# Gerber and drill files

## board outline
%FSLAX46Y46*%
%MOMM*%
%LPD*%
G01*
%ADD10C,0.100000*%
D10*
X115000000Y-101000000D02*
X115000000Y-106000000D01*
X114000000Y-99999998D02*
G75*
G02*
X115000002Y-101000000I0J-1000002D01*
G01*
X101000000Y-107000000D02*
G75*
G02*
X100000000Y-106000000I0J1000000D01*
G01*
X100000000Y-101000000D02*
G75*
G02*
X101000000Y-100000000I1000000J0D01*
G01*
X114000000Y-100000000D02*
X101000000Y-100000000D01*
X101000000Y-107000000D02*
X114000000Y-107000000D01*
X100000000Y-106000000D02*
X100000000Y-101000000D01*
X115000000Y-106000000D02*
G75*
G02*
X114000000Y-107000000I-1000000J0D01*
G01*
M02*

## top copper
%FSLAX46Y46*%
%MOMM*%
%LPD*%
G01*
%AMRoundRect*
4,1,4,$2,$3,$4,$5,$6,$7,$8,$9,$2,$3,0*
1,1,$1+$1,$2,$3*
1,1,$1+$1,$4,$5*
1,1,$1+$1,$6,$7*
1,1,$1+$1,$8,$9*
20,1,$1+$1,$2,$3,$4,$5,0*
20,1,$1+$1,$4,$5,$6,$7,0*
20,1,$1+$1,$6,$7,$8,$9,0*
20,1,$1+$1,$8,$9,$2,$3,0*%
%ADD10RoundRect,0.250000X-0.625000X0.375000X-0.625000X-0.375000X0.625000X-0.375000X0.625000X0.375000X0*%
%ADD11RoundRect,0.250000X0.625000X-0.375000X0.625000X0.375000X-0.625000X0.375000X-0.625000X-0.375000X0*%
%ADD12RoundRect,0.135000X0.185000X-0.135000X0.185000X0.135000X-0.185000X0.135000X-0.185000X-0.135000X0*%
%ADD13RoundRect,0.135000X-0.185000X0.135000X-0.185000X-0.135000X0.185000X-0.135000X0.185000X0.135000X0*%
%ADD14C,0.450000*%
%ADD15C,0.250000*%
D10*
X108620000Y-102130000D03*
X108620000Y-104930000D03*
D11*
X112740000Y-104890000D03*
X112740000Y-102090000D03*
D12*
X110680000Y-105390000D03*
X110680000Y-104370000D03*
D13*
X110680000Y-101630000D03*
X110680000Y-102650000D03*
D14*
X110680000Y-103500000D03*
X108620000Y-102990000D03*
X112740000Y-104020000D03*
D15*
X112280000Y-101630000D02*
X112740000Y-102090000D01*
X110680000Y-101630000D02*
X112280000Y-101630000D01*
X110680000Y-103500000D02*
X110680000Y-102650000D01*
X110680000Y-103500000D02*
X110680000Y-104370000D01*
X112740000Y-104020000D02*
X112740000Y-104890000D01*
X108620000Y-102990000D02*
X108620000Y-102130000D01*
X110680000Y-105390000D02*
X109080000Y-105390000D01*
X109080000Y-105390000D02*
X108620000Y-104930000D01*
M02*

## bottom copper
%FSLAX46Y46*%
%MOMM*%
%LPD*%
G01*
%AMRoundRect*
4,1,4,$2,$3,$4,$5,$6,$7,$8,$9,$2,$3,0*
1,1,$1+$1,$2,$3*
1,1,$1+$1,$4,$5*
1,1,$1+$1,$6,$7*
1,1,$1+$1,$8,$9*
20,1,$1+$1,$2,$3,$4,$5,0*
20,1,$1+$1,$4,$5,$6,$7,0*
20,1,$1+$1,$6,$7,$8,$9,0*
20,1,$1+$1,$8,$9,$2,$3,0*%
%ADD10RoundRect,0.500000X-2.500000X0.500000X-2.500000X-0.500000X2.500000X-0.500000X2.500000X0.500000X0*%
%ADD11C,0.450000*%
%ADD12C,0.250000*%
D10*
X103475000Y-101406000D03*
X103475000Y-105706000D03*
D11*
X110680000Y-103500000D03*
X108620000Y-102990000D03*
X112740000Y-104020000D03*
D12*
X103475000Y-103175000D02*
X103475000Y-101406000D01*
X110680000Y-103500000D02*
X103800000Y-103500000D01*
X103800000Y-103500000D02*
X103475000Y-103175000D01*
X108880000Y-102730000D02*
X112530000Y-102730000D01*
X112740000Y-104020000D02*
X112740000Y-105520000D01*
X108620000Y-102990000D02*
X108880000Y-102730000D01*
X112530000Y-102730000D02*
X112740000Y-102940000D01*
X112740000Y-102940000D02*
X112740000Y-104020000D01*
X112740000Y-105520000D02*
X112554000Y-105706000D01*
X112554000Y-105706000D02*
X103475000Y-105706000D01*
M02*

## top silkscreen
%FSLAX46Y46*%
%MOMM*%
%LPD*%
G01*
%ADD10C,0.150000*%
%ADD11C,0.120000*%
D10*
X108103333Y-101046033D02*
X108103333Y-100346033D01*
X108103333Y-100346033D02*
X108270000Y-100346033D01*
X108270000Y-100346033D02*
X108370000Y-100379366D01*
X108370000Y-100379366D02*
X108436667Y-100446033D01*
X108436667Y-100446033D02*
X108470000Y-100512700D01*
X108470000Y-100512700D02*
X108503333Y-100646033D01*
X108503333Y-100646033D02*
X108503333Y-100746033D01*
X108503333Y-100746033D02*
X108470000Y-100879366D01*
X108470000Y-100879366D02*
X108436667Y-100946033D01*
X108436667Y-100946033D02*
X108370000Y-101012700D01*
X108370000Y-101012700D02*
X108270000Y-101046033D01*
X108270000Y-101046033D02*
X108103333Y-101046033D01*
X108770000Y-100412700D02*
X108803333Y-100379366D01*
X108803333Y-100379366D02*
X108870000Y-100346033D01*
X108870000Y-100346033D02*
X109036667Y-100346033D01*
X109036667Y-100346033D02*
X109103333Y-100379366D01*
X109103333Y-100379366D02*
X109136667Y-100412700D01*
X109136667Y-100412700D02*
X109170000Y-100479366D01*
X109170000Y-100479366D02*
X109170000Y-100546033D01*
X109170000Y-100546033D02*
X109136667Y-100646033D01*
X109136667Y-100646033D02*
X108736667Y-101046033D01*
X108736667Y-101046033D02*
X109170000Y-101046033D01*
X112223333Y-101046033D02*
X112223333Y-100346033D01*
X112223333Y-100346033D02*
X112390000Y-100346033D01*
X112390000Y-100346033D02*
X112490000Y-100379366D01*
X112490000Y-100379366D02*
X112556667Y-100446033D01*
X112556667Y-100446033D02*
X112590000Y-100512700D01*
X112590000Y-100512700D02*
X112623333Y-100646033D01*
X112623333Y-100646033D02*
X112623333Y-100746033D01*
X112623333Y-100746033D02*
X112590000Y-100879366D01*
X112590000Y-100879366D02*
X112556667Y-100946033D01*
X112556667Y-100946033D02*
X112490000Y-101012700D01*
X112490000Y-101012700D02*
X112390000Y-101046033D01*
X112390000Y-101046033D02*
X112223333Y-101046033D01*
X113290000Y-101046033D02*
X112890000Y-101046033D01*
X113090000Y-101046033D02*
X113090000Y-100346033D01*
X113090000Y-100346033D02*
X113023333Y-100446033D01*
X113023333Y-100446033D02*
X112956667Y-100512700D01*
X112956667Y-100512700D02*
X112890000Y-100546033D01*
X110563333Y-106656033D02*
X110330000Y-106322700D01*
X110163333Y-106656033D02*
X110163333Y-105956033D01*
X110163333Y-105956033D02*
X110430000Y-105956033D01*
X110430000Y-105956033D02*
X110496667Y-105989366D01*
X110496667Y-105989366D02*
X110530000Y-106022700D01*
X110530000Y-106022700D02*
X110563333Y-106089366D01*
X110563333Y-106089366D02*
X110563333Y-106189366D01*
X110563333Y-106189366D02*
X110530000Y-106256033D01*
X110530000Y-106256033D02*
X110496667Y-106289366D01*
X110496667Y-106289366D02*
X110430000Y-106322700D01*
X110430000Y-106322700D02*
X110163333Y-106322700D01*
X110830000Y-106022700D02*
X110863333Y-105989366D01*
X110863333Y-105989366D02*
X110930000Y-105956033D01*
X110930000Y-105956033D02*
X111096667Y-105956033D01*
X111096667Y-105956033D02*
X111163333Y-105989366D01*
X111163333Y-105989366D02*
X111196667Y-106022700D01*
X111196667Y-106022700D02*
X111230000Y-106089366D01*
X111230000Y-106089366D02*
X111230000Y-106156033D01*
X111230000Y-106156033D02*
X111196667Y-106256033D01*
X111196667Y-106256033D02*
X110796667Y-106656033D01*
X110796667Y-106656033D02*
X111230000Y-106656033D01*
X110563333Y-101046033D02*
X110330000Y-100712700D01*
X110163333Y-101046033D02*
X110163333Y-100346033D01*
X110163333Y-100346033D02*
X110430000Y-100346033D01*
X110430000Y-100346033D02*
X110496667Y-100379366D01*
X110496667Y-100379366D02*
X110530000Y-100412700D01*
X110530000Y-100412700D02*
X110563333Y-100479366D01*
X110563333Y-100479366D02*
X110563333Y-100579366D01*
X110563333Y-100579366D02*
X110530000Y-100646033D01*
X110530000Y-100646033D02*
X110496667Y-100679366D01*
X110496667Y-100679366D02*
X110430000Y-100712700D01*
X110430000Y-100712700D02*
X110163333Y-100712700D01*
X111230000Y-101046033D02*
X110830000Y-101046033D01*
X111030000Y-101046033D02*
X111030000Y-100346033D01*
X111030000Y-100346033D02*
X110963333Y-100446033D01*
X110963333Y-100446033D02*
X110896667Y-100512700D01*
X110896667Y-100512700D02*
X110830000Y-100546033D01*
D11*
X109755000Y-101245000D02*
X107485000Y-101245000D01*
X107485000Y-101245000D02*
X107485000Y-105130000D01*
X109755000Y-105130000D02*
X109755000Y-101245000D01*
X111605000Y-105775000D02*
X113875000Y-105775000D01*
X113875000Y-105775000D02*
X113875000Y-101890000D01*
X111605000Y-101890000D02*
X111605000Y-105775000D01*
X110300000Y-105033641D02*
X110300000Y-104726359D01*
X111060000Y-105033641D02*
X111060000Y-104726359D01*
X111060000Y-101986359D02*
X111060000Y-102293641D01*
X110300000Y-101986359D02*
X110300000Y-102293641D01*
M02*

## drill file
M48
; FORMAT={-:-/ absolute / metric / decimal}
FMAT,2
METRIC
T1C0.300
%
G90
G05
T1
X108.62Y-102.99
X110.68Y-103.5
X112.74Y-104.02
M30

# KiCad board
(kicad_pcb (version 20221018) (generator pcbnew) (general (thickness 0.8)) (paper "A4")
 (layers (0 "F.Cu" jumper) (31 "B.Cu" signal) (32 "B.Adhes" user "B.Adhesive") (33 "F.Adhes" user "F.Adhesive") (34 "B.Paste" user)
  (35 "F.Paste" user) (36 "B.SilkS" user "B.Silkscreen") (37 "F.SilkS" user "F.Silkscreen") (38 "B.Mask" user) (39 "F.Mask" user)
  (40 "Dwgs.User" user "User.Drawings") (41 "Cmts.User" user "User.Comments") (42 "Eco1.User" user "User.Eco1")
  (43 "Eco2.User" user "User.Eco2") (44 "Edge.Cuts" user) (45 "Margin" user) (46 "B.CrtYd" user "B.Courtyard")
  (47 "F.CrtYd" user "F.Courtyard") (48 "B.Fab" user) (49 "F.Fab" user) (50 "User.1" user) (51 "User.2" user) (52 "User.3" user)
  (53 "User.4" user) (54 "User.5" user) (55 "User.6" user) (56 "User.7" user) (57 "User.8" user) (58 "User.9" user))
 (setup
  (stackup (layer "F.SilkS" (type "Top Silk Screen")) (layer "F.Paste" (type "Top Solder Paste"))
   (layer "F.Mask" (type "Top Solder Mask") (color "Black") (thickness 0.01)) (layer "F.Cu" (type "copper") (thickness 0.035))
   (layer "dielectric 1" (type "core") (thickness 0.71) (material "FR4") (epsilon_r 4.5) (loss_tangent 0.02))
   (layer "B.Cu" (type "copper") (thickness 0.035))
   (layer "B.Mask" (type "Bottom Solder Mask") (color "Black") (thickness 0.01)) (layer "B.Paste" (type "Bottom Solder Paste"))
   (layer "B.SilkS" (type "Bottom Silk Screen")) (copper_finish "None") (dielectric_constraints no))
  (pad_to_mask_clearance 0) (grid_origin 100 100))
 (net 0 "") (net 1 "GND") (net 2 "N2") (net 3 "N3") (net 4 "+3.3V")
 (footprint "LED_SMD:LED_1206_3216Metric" (layer "F.Cu") (at 108.62 103.53 -90)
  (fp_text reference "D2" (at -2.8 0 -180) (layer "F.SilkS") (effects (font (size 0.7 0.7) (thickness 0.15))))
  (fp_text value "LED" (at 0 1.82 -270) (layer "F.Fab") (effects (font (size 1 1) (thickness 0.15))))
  (fp_line (start -2.285 -1.135) (end -2.285 1.135) (stroke (width 0.12) (type solid)) (layer "F.SilkS"))
  (fp_line (start -2.285 1.135) (end 1.6 1.135) (stroke (width 0.12) (type solid)) (layer "F.SilkS"))
  (fp_line (start 1.6 -1.135) (end -2.285 -1.135) (stroke (width 0.12) (type solid)) (layer "F.SilkS"))
  (pad "1" smd roundrect (at -1.4 0 270) (size 1.25 1.75) (layers "F.Cu" "F.Paste" "F.Mask") (roundrect_rratio 0.2) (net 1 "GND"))
  (pad "2" smd roundrect (at 1.4 0 270) (size 1.25 1.75) (layers "F.Cu" "F.Paste" "F.Mask") (roundrect_rratio 0.2) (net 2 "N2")))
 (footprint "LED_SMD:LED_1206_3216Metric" (layer "F.Cu") (at 112.74 103.49 90)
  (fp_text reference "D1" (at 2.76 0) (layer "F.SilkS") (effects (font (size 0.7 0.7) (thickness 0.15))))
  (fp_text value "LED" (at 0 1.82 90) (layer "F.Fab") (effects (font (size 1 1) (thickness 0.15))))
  (fp_line (start -2.285 -1.135) (end -2.285 1.135) (stroke (width 0.12) (type solid)) (layer "F.SilkS"))
  (fp_line (start -2.285 1.135) (end 1.6 1.135) (stroke (width 0.12) (type solid)) (layer "F.SilkS"))
  (fp_line (start 1.6 -1.135) (end -2.285 -1.135) (stroke (width 0.12) (type solid)) (layer "F.SilkS"))
  (pad "1" smd roundrect (at -1.4 0 90) (size 1.25 1.75) (layers "F.Cu" "F.Paste" "F.Mask") (roundrect_rratio 0.2) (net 1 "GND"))
  (pad "2" smd roundrect (at 1.4 0 90) (size 1.25 1.75) (layers "F.Cu" "F.Paste" "F.Mask") (roundrect_rratio 0.2) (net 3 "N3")))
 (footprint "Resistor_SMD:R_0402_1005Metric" (layer "F.Cu") (at 110.68 104.88 90)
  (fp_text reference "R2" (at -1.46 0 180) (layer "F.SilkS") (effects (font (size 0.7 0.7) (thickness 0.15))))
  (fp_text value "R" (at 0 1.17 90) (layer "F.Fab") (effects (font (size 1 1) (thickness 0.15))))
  (fp_line (start -0.153641 -0.38) (end 0.153641 -0.38) (stroke (width 0.12) (type solid)) (layer "F.SilkS"))
  (fp_line (start -0.153641 0.38) (end 0.153641 0.38) (stroke (width 0.12) (type solid)) (layer "F.SilkS"))
  (pad "1" smd roundrect (at -0.51 0 90) (size 0.54 0.64) (layers "F.Cu" "F.Paste" "F.Mask") (roundrect_rratio 0.25) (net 2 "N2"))
  (pad "2" smd roundrect (at 0.51 0 90) (size 0.54 0.64) (layers "F.Cu" "F.Paste" "F.Mask") (roundrect_rratio 0.25) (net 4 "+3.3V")))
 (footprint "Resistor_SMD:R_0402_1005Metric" (layer "F.Cu") (at 110.68 102.14 -90)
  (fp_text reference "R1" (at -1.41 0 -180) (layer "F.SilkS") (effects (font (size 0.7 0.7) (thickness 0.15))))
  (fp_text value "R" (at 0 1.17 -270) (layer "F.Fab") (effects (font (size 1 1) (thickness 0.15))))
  (fp_line (start -0.153641 -0.38) (end 0.153641 -0.38) (stroke (width 0.12) (type solid)) (layer "F.SilkS"))
  (fp_line (start -0.153641 0.38) (end 0.153641 0.38) (stroke (width 0.12) (type solid)) (layer "F.SilkS"))
  (pad "1" smd roundrect (at -0.51 0 270) (size 0.54 0.64) (layers "F.Cu" "F.Paste" "F.Mask") (roundrect_rratio 0.25) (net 3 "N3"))
  (pad "2" smd roundrect (at 0.51 0 270) (size 0.54 0.64) (layers "F.Cu" "F.Paste" "F.Mask") (roundrect_rratio 0.25) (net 4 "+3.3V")))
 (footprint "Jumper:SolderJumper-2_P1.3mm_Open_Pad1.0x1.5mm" (layer "B.Cu") (at 103.475 103.556 -90)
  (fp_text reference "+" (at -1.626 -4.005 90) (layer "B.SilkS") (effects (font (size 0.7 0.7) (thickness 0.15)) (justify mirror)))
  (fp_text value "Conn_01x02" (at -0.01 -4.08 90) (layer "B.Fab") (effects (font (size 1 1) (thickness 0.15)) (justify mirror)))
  (pad "1" smd roundrect (at -2.15 0 270) (size 2 6) (layers "B.Cu" "B.Mask") (roundrect_rratio 0.25) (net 4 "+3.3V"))
  (pad "2" smd roundrect (at 2.15 0 270) (size 2 6) (layers "B.Cu" "B.Mask") (roundrect_rratio 0.25) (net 1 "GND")))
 (gr_line (start 115 101) (end 115 106) (stroke (width 0.1) (type default)) (layer "Edge.Cuts"))
 (gr_arc (start 114 99.999998) (mid 114.707107 100.292892) (end 115 101) (stroke (width 0.1) (type default)) (layer "Edge.Cuts"))
 (gr_arc (start 101 107) (mid 100.292894 106.707107) (end 100 106) (stroke (width 0.1) (type default)) (layer "Edge.Cuts"))
 (gr_arc (start 100 101) (mid 100.292893 100.292894) (end 101 100.000002) (stroke (width 0.1) (type default)) (layer "Edge.Cuts"))
 (gr_line (start 114 100) (end 101 100) (stroke (width 0.1) (type default)) (layer "Edge.Cuts"))
 (gr_line (start 101 107) (end 114 107) (stroke (width 0.1) (type default)) (layer "Edge.Cuts"))
 (gr_line (start 100 106) (end 100 101) (stroke (width 0.1) (type default)) (layer "Edge.Cuts"))
 (gr_arc (start 115 106) (mid 114.707106 106.707106) (end 114 107) (stroke (width 0.1) (type default)) (layer "Edge.Cuts"))
 (segment (start 112.28 101.63) (end 112.74 102.09) (width 0.25) (layer "F.Cu") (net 3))
 (segment (start 110.68 101.63) (end 112.28 101.63) (width 0.25) (layer "F.Cu") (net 3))
 (segment (start 110.68 103.5) (end 110.68 102.65) (width 0.25) (layer "F.Cu") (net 4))
 (segment (start 110.68 103.5) (end 110.68 104.37) (width 0.25) (layer "F.Cu") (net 4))
 (via (at 110.68 103.5) (size 0.45) (drill 0.3) (layers "F.Cu" "B.Cu") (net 4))
 (segment (start 103.475 103.175) (end 103.475 101.406) (width 0.25) (layer "B.Cu") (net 4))
 (segment (start 110.68 103.5) (end 103.8 103.5) (width 0.25) (layer "B.Cu") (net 4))
 (segment (start 103.8 103.5) (end 103.475 103.175) (width 0.25) (layer "B.Cu") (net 4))
 (segment (start 112.74 104.02) (end 112.74 104.89) (width 0.25) (layer "F.Cu") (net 1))
 (segment (start 108.62 102.99) (end 108.62 102.13) (width 0.25) (layer "F.Cu") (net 1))
 (via (at 108.62 102.99) (size 0.45) (drill 0.3) (layers "F.Cu" "B.Cu") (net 1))
 (via (at 112.74 104.02) (size 0.45) (drill 0.3) (layers "F.Cu" "B.Cu") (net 1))
 (segment (start 108.88 102.73) (end 112.53 102.73) (width 0.25) (layer "B.Cu") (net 1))
 (segment (start 112.74 104.02) (end 112.74 105.52) (width 0.25) (layer "B.Cu") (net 1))
 (segment (start 108.62 102.99) (end 108.88 102.73) (width 0.25) (layer "B.Cu") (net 1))
 (segment (start 112.53 102.73) (end 112.74 102.94) (width 0.25) (layer "B.Cu") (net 1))
 (segment (start 112.74 102.94) (end 112.74 104.02) (width 0.25) (layer "B.Cu") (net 1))
 (segment (start 112.74 105.52) (end 112.554 105.706) (width 0.25) (layer "B.Cu") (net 1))
 (segment (start 112.554 105.706) (end 103.475 105.706) (width 0.25) (layer "B.Cu") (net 1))
 (segment (start 110.68 105.39) (end 109.08 105.39) (width 0.25) (layer "F.Cu") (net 2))
 (segment (start 109.08 105.39) (end 108.62 104.93) (width 0.25) (layer "F.Cu") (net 2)))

